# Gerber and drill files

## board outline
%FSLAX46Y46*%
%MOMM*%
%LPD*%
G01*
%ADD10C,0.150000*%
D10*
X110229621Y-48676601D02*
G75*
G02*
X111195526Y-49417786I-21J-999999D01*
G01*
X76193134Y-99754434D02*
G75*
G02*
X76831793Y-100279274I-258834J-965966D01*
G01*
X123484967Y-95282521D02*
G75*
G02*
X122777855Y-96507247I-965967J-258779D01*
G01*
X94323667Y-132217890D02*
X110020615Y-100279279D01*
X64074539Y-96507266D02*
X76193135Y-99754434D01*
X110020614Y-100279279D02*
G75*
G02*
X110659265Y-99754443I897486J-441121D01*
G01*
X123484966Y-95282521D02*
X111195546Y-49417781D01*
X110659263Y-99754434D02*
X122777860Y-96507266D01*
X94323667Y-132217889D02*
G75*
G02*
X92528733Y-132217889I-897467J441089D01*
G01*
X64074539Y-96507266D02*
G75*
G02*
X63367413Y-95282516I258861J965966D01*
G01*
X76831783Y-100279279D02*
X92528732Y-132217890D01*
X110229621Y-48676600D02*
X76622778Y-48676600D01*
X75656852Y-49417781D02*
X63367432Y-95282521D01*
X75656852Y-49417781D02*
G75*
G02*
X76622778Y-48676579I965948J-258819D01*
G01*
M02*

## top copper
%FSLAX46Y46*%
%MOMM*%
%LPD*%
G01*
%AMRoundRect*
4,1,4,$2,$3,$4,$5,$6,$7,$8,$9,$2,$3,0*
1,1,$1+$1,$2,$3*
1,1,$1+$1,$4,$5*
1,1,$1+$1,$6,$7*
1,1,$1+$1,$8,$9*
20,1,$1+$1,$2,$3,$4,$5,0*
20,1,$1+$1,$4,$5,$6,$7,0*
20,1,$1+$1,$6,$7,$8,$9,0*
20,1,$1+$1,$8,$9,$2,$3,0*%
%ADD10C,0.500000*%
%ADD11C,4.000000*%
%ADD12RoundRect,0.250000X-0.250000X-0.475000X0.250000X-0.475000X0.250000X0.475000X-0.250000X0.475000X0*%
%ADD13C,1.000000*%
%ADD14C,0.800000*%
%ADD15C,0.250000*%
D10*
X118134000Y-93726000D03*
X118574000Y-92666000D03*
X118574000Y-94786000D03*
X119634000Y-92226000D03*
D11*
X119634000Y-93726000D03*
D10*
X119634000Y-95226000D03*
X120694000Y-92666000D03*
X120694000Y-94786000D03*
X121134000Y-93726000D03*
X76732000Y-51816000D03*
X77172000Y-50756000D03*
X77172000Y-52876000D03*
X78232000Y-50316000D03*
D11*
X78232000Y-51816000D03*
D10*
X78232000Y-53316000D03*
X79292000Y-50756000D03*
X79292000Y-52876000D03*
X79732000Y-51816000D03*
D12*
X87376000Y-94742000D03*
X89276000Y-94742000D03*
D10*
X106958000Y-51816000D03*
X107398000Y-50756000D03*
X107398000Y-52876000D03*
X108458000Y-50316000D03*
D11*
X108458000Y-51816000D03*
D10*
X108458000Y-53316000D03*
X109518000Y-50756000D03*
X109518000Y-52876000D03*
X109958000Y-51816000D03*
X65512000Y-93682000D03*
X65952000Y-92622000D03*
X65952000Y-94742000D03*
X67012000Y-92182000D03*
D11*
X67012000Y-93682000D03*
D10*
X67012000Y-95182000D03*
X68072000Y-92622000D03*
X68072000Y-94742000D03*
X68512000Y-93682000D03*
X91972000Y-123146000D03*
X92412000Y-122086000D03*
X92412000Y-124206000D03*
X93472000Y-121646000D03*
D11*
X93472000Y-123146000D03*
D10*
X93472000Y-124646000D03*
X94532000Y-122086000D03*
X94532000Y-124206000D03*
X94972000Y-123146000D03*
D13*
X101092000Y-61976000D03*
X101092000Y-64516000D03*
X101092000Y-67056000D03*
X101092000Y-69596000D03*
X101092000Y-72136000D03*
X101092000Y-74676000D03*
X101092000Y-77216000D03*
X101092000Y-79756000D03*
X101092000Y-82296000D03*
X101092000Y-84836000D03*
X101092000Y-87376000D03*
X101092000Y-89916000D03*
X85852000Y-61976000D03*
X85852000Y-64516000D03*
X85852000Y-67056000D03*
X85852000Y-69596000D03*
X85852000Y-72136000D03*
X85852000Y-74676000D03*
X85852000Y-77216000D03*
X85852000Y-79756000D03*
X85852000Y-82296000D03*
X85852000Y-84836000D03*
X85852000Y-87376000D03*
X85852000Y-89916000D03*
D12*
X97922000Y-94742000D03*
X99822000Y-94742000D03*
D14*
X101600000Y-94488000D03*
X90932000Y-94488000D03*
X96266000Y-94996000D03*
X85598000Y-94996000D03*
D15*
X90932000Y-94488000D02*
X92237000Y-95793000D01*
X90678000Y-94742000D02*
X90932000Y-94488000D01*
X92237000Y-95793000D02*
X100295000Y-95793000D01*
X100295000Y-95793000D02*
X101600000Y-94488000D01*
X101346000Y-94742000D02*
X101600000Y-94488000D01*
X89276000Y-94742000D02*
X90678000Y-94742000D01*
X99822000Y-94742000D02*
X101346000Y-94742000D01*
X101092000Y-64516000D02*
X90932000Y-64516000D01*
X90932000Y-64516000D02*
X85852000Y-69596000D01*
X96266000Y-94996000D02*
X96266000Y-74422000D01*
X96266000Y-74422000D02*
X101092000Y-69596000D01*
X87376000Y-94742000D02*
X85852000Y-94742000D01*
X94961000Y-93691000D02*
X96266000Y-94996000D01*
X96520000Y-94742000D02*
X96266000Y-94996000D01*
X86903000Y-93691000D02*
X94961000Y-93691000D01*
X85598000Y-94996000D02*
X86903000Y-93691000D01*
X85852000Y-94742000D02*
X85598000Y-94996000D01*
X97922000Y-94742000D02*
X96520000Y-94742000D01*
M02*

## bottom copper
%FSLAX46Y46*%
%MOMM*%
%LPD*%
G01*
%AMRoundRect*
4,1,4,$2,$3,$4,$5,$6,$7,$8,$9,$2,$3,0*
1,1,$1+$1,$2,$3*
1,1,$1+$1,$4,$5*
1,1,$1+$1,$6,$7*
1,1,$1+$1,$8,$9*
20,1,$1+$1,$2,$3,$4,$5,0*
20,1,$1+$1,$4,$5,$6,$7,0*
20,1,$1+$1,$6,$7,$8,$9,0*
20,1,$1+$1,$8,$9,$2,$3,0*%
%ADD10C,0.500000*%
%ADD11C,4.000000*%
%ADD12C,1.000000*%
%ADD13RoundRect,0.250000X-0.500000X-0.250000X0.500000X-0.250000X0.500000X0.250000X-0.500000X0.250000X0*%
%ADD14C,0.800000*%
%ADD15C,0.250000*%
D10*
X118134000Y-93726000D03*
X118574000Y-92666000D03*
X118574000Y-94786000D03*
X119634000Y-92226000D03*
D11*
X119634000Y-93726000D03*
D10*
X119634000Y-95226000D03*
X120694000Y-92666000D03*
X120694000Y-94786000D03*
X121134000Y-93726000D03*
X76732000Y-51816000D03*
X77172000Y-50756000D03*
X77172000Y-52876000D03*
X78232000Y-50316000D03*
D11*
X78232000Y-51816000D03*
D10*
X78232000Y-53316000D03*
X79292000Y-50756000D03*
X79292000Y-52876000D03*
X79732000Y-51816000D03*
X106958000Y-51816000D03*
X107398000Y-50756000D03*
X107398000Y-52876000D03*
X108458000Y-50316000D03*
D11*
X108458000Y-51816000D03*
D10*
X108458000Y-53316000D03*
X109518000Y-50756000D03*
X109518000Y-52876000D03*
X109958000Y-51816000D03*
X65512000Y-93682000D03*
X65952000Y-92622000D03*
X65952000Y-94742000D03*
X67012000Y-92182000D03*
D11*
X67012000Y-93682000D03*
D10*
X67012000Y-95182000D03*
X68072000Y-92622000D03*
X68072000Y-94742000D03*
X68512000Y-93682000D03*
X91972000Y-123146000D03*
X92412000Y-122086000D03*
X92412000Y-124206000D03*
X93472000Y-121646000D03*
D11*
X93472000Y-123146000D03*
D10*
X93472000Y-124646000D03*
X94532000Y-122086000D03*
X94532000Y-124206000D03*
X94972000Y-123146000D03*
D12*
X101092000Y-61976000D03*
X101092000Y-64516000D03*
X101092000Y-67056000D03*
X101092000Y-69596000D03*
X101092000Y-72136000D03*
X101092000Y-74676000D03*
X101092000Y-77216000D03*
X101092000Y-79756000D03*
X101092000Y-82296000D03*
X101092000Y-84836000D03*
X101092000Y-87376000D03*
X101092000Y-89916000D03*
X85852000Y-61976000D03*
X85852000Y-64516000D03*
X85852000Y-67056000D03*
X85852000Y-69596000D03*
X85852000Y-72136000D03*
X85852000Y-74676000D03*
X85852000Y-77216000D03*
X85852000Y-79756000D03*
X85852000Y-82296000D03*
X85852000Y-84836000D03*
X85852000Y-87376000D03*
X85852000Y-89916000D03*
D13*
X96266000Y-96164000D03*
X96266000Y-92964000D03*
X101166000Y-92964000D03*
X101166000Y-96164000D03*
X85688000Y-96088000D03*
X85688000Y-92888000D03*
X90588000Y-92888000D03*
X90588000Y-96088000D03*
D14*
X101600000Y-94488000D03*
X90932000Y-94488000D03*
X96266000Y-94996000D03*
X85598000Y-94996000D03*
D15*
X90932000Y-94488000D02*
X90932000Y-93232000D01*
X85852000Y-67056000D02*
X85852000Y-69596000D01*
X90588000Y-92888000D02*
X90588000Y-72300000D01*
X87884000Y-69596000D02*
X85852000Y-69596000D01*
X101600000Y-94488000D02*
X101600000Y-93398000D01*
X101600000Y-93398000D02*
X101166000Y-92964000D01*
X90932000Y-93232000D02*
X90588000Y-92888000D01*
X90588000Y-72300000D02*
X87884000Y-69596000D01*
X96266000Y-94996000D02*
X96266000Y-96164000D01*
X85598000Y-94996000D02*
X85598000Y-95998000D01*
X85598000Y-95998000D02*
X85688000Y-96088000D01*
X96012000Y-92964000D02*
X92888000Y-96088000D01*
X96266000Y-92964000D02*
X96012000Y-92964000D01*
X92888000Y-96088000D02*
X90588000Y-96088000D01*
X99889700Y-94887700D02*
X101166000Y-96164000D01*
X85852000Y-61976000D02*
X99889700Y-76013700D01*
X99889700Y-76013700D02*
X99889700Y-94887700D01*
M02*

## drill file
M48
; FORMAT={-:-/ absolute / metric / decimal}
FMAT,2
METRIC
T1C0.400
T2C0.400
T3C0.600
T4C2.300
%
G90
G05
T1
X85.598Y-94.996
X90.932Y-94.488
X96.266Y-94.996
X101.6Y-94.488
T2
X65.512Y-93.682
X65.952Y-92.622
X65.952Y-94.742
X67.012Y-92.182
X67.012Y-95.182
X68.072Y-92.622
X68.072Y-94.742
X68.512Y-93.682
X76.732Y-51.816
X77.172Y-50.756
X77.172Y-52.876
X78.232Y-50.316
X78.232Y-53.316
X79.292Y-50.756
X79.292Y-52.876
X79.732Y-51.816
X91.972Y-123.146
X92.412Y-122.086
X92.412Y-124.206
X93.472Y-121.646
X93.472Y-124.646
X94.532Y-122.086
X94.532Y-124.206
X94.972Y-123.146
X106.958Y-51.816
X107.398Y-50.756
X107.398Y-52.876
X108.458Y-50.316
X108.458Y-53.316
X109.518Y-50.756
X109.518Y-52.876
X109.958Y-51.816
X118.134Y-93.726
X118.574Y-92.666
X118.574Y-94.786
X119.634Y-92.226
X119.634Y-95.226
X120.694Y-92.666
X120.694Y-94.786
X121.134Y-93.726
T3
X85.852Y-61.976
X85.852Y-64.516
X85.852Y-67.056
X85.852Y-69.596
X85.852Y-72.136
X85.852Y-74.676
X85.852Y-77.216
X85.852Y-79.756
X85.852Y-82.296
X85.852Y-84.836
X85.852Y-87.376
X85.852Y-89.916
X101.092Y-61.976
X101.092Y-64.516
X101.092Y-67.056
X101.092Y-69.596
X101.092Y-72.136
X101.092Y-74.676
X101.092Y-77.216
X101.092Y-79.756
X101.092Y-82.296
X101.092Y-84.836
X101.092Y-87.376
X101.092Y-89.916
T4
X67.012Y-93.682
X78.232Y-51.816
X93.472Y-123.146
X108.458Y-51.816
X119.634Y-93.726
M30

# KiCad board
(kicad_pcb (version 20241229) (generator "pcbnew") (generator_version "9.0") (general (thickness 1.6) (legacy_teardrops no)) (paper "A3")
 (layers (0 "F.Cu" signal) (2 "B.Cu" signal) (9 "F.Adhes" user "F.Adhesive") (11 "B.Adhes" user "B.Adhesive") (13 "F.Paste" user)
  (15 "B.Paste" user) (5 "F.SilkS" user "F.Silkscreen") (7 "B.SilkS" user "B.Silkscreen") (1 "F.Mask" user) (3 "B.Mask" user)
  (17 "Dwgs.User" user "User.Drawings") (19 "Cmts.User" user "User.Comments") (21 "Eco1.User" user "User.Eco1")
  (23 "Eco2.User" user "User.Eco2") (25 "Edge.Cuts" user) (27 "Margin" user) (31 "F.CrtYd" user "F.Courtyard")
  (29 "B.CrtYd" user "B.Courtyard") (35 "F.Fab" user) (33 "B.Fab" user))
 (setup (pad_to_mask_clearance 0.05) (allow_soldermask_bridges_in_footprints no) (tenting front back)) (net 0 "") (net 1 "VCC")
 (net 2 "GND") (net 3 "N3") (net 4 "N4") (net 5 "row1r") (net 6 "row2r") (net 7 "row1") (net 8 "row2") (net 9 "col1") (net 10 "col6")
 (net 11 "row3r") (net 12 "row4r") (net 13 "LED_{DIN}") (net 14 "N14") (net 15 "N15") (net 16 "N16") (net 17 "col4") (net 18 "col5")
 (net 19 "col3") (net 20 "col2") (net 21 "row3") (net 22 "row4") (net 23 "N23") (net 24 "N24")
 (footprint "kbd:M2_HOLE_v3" (layer "F.Cu") (at 119.634 93.726)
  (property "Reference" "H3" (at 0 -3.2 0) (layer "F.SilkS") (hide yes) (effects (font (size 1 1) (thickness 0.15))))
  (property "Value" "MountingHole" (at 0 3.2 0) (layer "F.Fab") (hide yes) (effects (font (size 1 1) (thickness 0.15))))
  (pad "1" thru_hole circle (at -1.5 0) (size 0.5 0.5) (drill 0.4) (layers "*.Cu" "*.Mask") (remove_unused_layers no))
  (pad "1" thru_hole circle (at -1.06 -1.06) (size 0.5 0.5) (drill 0.4) (layers "*.Cu" "*.Mask") (remove_unused_layers no))
  (pad "1" thru_hole circle (at -1.06 1.06) (size 0.5 0.5) (drill 0.4) (layers "*.Cu" "*.Mask") (remove_unused_layers no))
  (pad "1" thru_hole circle (at 0 -1.5) (size 0.5 0.5) (drill 0.4) (layers "*.Cu" "*.Mask") (remove_unused_layers no))
  (pad "1" thru_hole circle (at 0 0) (size 4 4) (drill 2.3) (layers "*.Cu" "*.Mask") (remove_unused_layers no))
  (pad "1" thru_hole circle (at 0 1.5) (size 0.5 0.5) (drill 0.4) (layers "*.Cu" "*.Mask") (remove_unused_layers no))
  (pad "1" thru_hole circle (at 1.06 -1.06) (size 0.5 0.5) (drill 0.4) (layers "*.Cu" "*.Mask") (remove_unused_layers no))
  (pad "1" thru_hole circle (at 1.06 1.06) (size 0.5 0.5) (drill 0.4) (layers "*.Cu" "*.Mask") (remove_unused_layers no))
  (pad "1" thru_hole circle (at 1.5 0) (size 0.5 0.5) (drill 0.4) (layers "*.Cu" "*.Mask") (remove_unused_layers no)))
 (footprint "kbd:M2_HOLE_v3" (layer "F.Cu") (at 78.232 51.816)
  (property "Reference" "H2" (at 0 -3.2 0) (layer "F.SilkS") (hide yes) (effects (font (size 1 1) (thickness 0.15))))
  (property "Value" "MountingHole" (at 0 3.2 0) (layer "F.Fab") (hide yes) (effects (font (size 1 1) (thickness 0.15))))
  (pad "1" thru_hole circle (at -1.5 0) (size 0.5 0.5) (drill 0.4) (layers "*.Cu" "*.Mask") (remove_unused_layers no))
  (pad "1" thru_hole circle (at -1.06 -1.06) (size 0.5 0.5) (drill 0.4) (layers "*.Cu" "*.Mask") (remove_unused_layers no))
  (pad "1" thru_hole circle (at -1.06 1.06) (size 0.5 0.5) (drill 0.4) (layers "*.Cu" "*.Mask") (remove_unused_layers no))
  (pad "1" thru_hole circle (at 0 -1.5) (size 0.5 0.5) (drill 0.4) (layers "*.Cu" "*.Mask") (remove_unused_layers no))
  (pad "1" thru_hole circle (at 0 0) (size 4 4) (drill 2.3) (layers "*.Cu" "*.Mask") (remove_unused_layers no))
  (pad "1" thru_hole circle (at 0 1.5) (size 0.5 0.5) (drill 0.4) (layers "*.Cu" "*.Mask") (remove_unused_layers no))
  (pad "1" thru_hole circle (at 1.06 -1.06) (size 0.5 0.5) (drill 0.4) (layers "*.Cu" "*.Mask") (remove_unused_layers no))
  (pad "1" thru_hole circle (at 1.06 1.06) (size 0.5 0.5) (drill 0.4) (layers "*.Cu" "*.Mask") (remove_unused_layers no))
  (pad "1" thru_hole circle (at 1.5 0) (size 0.5 0.5) (drill 0.4) (layers "*.Cu" "*.Mask") (remove_unused_layers no)))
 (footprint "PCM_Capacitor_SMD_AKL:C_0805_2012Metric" (layer "F.Cu") (at 88.326 94.742)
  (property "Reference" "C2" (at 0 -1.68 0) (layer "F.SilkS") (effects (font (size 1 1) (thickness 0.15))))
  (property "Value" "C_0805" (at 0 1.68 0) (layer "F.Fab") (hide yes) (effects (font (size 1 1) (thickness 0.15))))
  (pad "1" smd roundrect (at -0.95 0) (size 1 1.45) (layers "F.Cu" "F.Mask" "F.Paste") (roundrect_rratio 0.25) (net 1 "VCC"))
  (pad "2" smd roundrect (at 0.95 0) (size 1 1.45) (layers "F.Cu" "F.Mask" "F.Paste") (roundrect_rratio 0.25) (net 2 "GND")))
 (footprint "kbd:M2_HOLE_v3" (layer "F.Cu") (at 108.458 51.816)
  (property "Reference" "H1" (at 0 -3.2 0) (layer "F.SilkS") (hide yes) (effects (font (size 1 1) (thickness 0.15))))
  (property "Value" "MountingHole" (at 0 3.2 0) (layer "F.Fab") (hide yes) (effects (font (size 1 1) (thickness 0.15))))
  (pad "1" thru_hole circle (at -1.5 0) (size 0.5 0.5) (drill 0.4) (layers "*.Cu" "*.Mask") (remove_unused_layers no))
  (pad "1" thru_hole circle (at -1.06 -1.06) (size 0.5 0.5) (drill 0.4) (layers "*.Cu" "*.Mask") (remove_unused_layers no))
  (pad "1" thru_hole circle (at -1.06 1.06) (size 0.5 0.5) (drill 0.4) (layers "*.Cu" "*.Mask") (remove_unused_layers no))
  (pad "1" thru_hole circle (at 0 -1.5) (size 0.5 0.5) (drill 0.4) (layers "*.Cu" "*.Mask") (remove_unused_layers no))
  (pad "1" thru_hole circle (at 0 0) (size 4 4) (drill 2.3) (layers "*.Cu" "*.Mask") (remove_unused_layers no))
  (pad "1" thru_hole circle (at 0 1.5) (size 0.5 0.5) (drill 0.4) (layers "*.Cu" "*.Mask") (remove_unused_layers no))
  (pad "1" thru_hole circle (at 1.06 -1.06) (size 0.5 0.5) (drill 0.4) (layers "*.Cu" "*.Mask") (remove_unused_layers no))
  (pad "1" thru_hole circle (at 1.06 1.06) (size 0.5 0.5) (drill 0.4) (layers "*.Cu" "*.Mask") (remove_unused_layers no))
  (pad "1" thru_hole circle (at 1.5 0) (size 0.5 0.5) (drill 0.4) (layers "*.Cu" "*.Mask") (remove_unused_layers no)))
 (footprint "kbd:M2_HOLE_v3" (layer "F.Cu") (at 67.012 93.682)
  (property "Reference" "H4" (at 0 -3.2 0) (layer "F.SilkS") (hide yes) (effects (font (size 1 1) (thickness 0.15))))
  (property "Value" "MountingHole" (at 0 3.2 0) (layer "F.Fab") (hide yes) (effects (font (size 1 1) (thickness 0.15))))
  (pad "1" thru_hole circle (at -1.5 0) (size 0.5 0.5) (drill 0.4) (layers "*.Cu" "*.Mask") (remove_unused_layers no))
  (pad "1" thru_hole circle (at -1.06 -1.06) (size 0.5 0.5) (drill 0.4) (layers "*.Cu" "*.Mask") (remove_unused_layers no))
  (pad "1" thru_hole circle (at -1.06 1.06) (size 0.5 0.5) (drill 0.4) (layers "*.Cu" "*.Mask") (remove_unused_layers no))
  (pad "1" thru_hole circle (at 0 -1.5) (size 0.5 0.5) (drill 0.4) (layers "*.Cu" "*.Mask") (remove_unused_layers no))
  (pad "1" thru_hole circle (at 0 0) (size 4 4) (drill 2.3) (layers "*.Cu" "*.Mask") (remove_unused_layers no))
  (pad "1" thru_hole circle (at 0 1.5) (size 0.5 0.5) (drill 0.4) (layers "*.Cu" "*.Mask") (remove_unused_layers no))
  (pad "1" thru_hole circle (at 1.06 -1.06) (size 0.5 0.5) (drill 0.4) (layers "*.Cu" "*.Mask") (remove_unused_layers no))
  (pad "1" thru_hole circle (at 1.06 1.06) (size 0.5 0.5) (drill 0.4) (layers "*.Cu" "*.Mask") (remove_unused_layers no))
  (pad "1" thru_hole circle (at 1.5 0) (size 0.5 0.5) (drill 0.4) (layers "*.Cu" "*.Mask") (remove_unused_layers no)))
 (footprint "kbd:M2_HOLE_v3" (layer "F.Cu") (at 93.472 123.146)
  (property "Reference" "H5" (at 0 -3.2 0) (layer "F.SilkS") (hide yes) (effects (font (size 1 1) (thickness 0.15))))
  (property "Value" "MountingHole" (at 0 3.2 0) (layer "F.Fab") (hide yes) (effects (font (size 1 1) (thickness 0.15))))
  (pad "1" thru_hole circle (at -1.5 0) (size 0.5 0.5) (drill 0.4) (layers "*.Cu" "*.Mask") (remove_unused_layers no))
  (pad "1" thru_hole circle (at -1.06 -1.06) (size 0.5 0.5) (drill 0.4) (layers "*.Cu" "*.Mask") (remove_unused_layers no))
  (pad "1" thru_hole circle (at -1.06 1.06) (size 0.5 0.5) (drill 0.4) (layers "*.Cu" "*.Mask") (remove_unused_layers no))
  (pad "1" thru_hole circle (at 0 -1.5) (size 0.5 0.5) (drill 0.4) (layers "*.Cu" "*.Mask") (remove_unused_layers no))
  (pad "1" thru_hole circle (at 0 0) (size 4 4) (drill 2.3) (layers "*.Cu" "*.Mask") (remove_unused_layers no))
  (pad "1" thru_hole circle (at 0 1.5) (size 0.5 0.5) (drill 0.4) (layers "*.Cu" "*.Mask") (remove_unused_layers no))
  (pad "1" thru_hole circle (at 1.06 -1.06) (size 0.5 0.5) (drill 0.4) (layers "*.Cu" "*.Mask") (remove_unused_layers no))
  (pad "1" thru_hole circle (at 1.06 1.06) (size 0.5 0.5) (drill 0.4) (layers "*.Cu" "*.Mask") (remove_unused_layers no))
  (pad "1" thru_hole circle (at 1.5 0) (size 0.5 0.5) (drill 0.4) (layers "*.Cu" "*.Mask") (remove_unused_layers no)))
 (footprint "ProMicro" (layer "F.Cu") (at 93.472 75.946 -90)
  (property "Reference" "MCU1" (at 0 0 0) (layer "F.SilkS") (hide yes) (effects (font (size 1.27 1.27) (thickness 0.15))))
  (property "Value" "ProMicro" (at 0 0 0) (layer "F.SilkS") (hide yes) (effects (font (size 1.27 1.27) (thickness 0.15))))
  (pad "1" thru_hole circle (at -13.97 -7.62) (size 1 1) (drill 0.6) (layers "*.Cu" "F.Mask" "F.SilkS") (remove_unused_layers no)
   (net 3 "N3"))
  (pad "2" thru_hole circle (at -11.43 -7.62) (size 1 1) (drill 0.6) (layers "*.Cu" "F.Mask" "F.SilkS") (remove_unused_layers no)
   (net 2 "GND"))
  (pad "3" thru_hole circle (at -8.89 -7.62) (size 1 1) (drill 0.6) (layers "*.Cu" "F.Mask" "F.SilkS") (remove_unused_layers no)
   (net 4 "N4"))
  (pad "4" thru_hole circle (at -6.35 -7.62) (size 1 1) (drill 0.6) (layers "*.Cu" "F.Mask" "F.SilkS") (remove_unused_layers no)
   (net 1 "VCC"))
  (pad "5" thru_hole circle (at -3.81 -7.62) (size 1 1) (drill 0.6) (layers "*.Cu" "F.Mask" "F.SilkS") (remove_unused_layers no)
   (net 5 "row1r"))
  (pad "6" thru_hole circle (at -1.27 -7.62) (size 1 1) (drill 0.6) (layers "*.Cu" "F.Mask" "F.SilkS") (remove_unused_layers no)
   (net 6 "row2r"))
  (pad "7" thru_hole circle (at 1.27 -7.62) (size 1 1) (drill 0.6) (layers "*.Cu" "F.Mask" "F.SilkS") (remove_unused_layers no)
   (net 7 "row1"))
  (pad "8" thru_hole circle (at 3.81 -7.62) (size 1 1) (drill 0.6) (layers "*.Cu" "F.Mask" "F.SilkS") (remove_unused_layers no)
   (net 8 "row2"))
  (pad "9" thru_hole circle (at 6.35 -7.62) (size 1 1) (drill 0.6) (layers "*.Cu" "F.Mask" "F.SilkS") (remove_unused_layers no)
   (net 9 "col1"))
  (pad "10" thru_hole circle (at 8.89 -7.62) (size 1 1) (drill 0.6) (layers "*.Cu" "F.Mask" "F.SilkS") (remove_unused_layers no)
   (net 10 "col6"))
  (pad "11" thru_hole circle (at 11.43 -7.62) (size 1 1) (drill 0.6) (layers "*.Cu" "F.Mask" "F.SilkS") (remove_unused_layers no)
   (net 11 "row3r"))
  (pad "12" thru_hole circle (at 13.97 -7.62) (size 1 1) (drill 0.6) (layers "*.Cu" "F.Mask" "F.SilkS") (remove_unused_layers no)
   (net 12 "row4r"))
  (pad "13" thru_hole circle (at -13.97 7.62) (size 1 1) (drill 0.6) (layers "*.Cu" "F.Mask" "F.SilkS") (remove_unused_layers no)
   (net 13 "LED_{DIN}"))
  (pad "14" thru_hole circle (at -11.43 7.62) (size 1 1) (drill 0.6) (layers "*.Cu" "F.Mask" "F.SilkS") (remove_unused_layers no)
   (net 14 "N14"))
  (pad "15" thru_hole circle (at -8.89 7.62) (size 1 1) (drill 0.6) (layers "*.Cu" "F.Mask" "F.SilkS") (remove_unused_layers no)
   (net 2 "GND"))
  (pad "16" thru_hole circle (at -6.35 7.62) (size 1 1) (drill 0.6) (layers "*.Cu" "F.Mask" "F.SilkS") (remove_unused_layers no)
   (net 2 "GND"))
  (pad "17" thru_hole circle (at -3.81 7.62) (size 1 1) (drill 0.6) (layers "*.Cu" "F.Mask" "F.SilkS") (remove_unused_layers no)
   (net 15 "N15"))
  (pad "18" thru_hole circle (at -1.27 7.62) (size 1 1) (drill 0.6) (layers "*.Cu" "F.Mask" "F.SilkS") (remove_unused_layers no)
   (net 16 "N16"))
  (pad "19" thru_hole circle (at 1.27 7.62) (size 1 1) (drill 0.6) (layers "*.Cu" "F.Mask" "F.SilkS") (remove_unused_layers no)
   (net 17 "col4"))
  (pad "20" thru_hole circle (at 3.81 7.62) (size 1 1) (drill 0.6) (layers "*.Cu" "F.Mask" "F.SilkS") (remove_unused_layers no)
   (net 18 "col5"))
  (pad "21" thru_hole circle (at 6.35 7.62) (size 1 1) (drill 0.6) (layers "*.Cu" "F.Mask" "F.SilkS") (remove_unused_layers no)
   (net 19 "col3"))
  (pad "22" thru_hole circle (at 8.89 7.62) (size 1 1) (drill 0.6) (layers "*.Cu" "F.Mask" "F.SilkS") (remove_unused_layers no)
   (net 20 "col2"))
  (pad "23" thru_hole circle (at 11.43 7.62) (size 1 1) (drill 0.6) (layers "*.Cu" "F.Mask" "F.SilkS") (remove_unused_layers no)
   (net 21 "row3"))
  (pad "24" thru_hole circle (at 13.97 7.62) (size 1 1) (drill 0.6) (layers "*.Cu" "F.Mask" "F.SilkS") (remove_unused_layers no)
   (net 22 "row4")))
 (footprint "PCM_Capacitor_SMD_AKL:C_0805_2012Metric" (layer "F.Cu") (at 98.872 94.742)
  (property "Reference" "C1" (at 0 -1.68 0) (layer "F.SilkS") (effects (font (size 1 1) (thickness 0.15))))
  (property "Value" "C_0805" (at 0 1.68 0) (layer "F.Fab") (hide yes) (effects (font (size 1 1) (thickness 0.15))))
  (pad "1" smd roundrect (at -0.95 0) (size 1 1.45) (layers "F.Cu" "F.Mask" "F.Paste") (roundrect_rratio 0.25) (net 1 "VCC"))
  (pad "2" smd roundrect (at 0.95 0) (size 1 1.45) (layers "F.Cu" "F.Mask" "F.Paste") (roundrect_rratio 0.25) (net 2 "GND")))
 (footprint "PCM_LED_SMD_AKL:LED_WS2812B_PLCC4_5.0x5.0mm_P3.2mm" (layer "B.Cu") (at 98.716 94.564)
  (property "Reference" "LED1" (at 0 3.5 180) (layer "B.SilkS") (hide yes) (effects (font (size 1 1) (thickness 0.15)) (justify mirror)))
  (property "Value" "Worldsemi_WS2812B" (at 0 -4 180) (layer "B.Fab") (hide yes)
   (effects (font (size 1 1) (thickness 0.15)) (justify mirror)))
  (pad "1" smd roundrect (at -2.45 1.6) (size 1.5 1) (layers "B.Cu" "B.Mask" "B.Paste") (roundrect_rratio 0.25) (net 1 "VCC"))
  (pad "2" smd roundrect (at -2.45 -1.6) (size 1.5 1) (layers "B.Cu" "B.Mask" "B.Paste") (roundrect_rratio 0.25) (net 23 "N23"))
  (pad "3" smd roundrect (at 2.45 -1.6) (size 1.5 1) (layers "B.Cu" "B.Mask" "B.Paste") (roundrect_rratio 0.25) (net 2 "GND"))
  (pad "4" smd roundrect (at 2.45 1.6) (size 1.5 1) (layers "B.Cu" "B.Mask" "B.Paste") (roundrect_rratio 0.25) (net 13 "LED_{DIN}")))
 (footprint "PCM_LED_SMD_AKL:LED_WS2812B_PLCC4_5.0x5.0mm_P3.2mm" (layer "B.Cu") (at 88.138 94.488)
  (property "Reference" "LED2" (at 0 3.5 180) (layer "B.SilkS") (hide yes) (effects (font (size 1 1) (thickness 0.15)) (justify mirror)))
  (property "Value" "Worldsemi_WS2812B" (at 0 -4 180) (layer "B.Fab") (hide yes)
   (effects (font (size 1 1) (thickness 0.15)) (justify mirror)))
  (pad "1" smd roundrect (at -2.45 1.6) (size 1.5 1) (layers "B.Cu" "B.Mask" "B.Paste") (roundrect_rratio 0.25) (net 1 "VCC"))
  (pad "2" smd roundrect (at -2.45 -1.6) (size 1.5 1) (layers "B.Cu" "B.Mask" "B.Paste") (roundrect_rratio 0.25) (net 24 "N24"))
  (pad "3" smd roundrect (at 2.45 -1.6) (size 1.5 1) (layers "B.Cu" "B.Mask" "B.Paste") (roundrect_rratio 0.25) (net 2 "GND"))
  (pad "4" smd roundrect (at 2.45 1.6) (size 1.5 1) (layers "B.Cu" "B.Mask" "B.Paste") (roundrect_rratio 0.25) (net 23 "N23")))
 (gr_arc (start 110.229621 48.676601) (mid 110.838382 48.883247) (end 111.195546 49.417781) (stroke (width 0.15) (type solid))
  (layer "Edge.Cuts"))
 (gr_arc (start 76.193134 99.754434) (mid 76.569229 99.947776) (end 76.831783 100.279279) (stroke (width 0.15) (type solid))
  (layer "Edge.Cuts"))
 (gr_arc (start 123.484967 95.282521) (mid 123.385066 96.04134) (end 122.77786 96.507266) (stroke (width 0.15) (type solid))
  (layer "Edge.Cuts"))
 (gr_line (start 94.323667 132.21789) (end 110.020615 100.279279) (stroke (width 0.15) (type solid)) (layer "Edge.Cuts"))
 (gr_line (start 64.074539 96.507266) (end 76.193135 99.754434) (stroke (width 0.15) (type solid)) (layer "Edge.Cuts"))
 (gr_arc (start 110.020614 100.279279) (mid 110.283168 99.947776) (end 110.659263 99.754434) (stroke (width 0.15) (type solid))
  (layer "Edge.Cuts"))
 (gr_line (start 123.484966 95.282521) (end 111.195546 49.417781) (stroke (width 0.15) (type solid)) (layer "Edge.Cuts"))
 (gr_line (start 110.659263 99.754434) (end 122.77786 96.507266) (stroke (width 0.15) (type solid)) (layer "Edge.Cuts"))
 (gr_arc (start 94.323667 132.217889) (mid 93.4262 132.776809) (end 92.528732 132.21789) (stroke (width 0.15) (type solid))
  (layer "Edge.Cuts"))
 (gr_arc (start 64.074539 96.507266) (mid 63.467333 96.04134) (end 63.367432 95.282521) (stroke (width 0.15) (type solid))
  (layer "Edge.Cuts"))
 (gr_line (start 76.831783 100.279279) (end 92.528732 132.21789) (stroke (width 0.15) (type solid)) (layer "Edge.Cuts"))
 (gr_line (start 110.229621 48.6766) (end 76.622778 48.6766) (stroke (width 0.15) (type solid)) (layer "Edge.Cuts"))
 (gr_line (start 75.656852 49.417781) (end 63.367432 95.282521) (stroke (width 0.15) (type solid)) (layer "Edge.Cuts"))
 (gr_arc (start 75.656852 49.417781) (mid 76.014016 48.883247) (end 76.622778 48.6766) (stroke (width 0.15) (type solid))
  (layer "Edge.Cuts"))
 (segment (start 90.932 94.488) (end 92.237 95.793) (width 0.25) (layer "F.Cu") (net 2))
 (segment (start 90.678 94.742) (end 90.932 94.488) (width 0.25) (layer "F.Cu") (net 2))
 (segment (start 92.237 95.793) (end 100.295 95.793) (width 0.25) (layer "F.Cu") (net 2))
 (segment (start 100.295 95.793) (end 101.6 94.488) (width 0.25) (layer "F.Cu") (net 2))
 (segment (start 101.346 94.742) (end 101.6 94.488) (width 0.25) (layer "F.Cu") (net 2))
 (segment (start 89.276 94.742) (end 90.678 94.742) (width 0.25) (layer "F.Cu") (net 2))
 (segment (start 99.822 94.742) (end 101.346 94.742) (width 0.25) (layer "F.Cu") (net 2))
 (segment (start 101.092 64.516) (end 90.932 64.516) (width 0.25) (layer "F.Cu") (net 2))
 (segment (start 90.932 64.516) (end 85.852 69.596) (width 0.25) (layer "F.Cu") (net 2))
 (via (at 101.6 94.488) (size 0.8) (drill 0.4) (layers "F.Cu" "B.Cu") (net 2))
 (via (at 90.932 94.488) (size 0.8) (drill 0.4) (layers "F.Cu" "B.Cu") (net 2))
 (segment (start 90.932 94.488) (end 90.932 93.232) (width 0.25) (layer "B.Cu") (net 2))
 (segment (start 85.852 67.056) (end 85.852 69.596) (width 0.25) (layer "B.Cu") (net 2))
 (segment (start 90.588 92.888) (end 90.588 72.3) (width 0.25) (layer "B.Cu") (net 2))
 (segment (start 87.884 69.596) (end 85.852 69.596) (width 0.25) (layer "B.Cu") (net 2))
 (segment (start 101.6 94.488) (end 101.6 93.398) (width 0.25) (layer "B.Cu") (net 2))
 (segment (start 101.6 93.398) (end 101.166 92.964) (width 0.25) (layer "B.Cu") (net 2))
 (segment (start 90.932 93.232) (end 90.588 92.888) (width 0.25) (layer "B.Cu") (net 2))
 (segment (start 90.588 72.3) (end 87.884 69.596) (width 0.25) (layer "B.Cu") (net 2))
 (segment (start 96.266 94.996) (end 96.266 74.422) (width 0.25) (layer "F.Cu") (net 1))
 (segment (start 96.266 74.422) (end 101.092 69.596) (width 0.25) (layer "F.Cu") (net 1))
 (segment (start 87.376 94.742) (end 85.852 94.742) (width 0.25) (layer "F.Cu") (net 1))
 (segment (start 94.961 93.691) (end 96.266 94.996) (width 0.25) (layer "F.Cu") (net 1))
 (segment (start 96.52 94.742) (end 96.266 94.996) (width 0.25) (layer "F.Cu") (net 1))
 (segment (start 86.903 93.691) (end 94.961 93.691) (width 0.25) (layer "F.Cu") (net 1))
 (segment (start 85.598 94.996) (end 86.903 93.691) (width 0.25) (layer "F.Cu") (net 1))
 (segment (start 85.852 94.742) (end 85.598 94.996) (width 0.25) (layer "F.Cu") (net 1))
 (segment (start 97.922 94.742) (end 96.52 94.742) (width 0.25) (layer "F.Cu") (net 1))
 (via (at 96.266 94.996) (size 0.8) (drill 0.4) (layers "F.Cu" "B.Cu") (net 1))
 (via (at 85.598 94.996) (size 0.8) (drill 0.4) (layers "F.Cu" "B.Cu") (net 1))
 (segment (start 96.266 94.996) (end 96.266 96.164) (width 0.25) (layer "B.Cu") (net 1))
 (segment (start 85.598 94.996) (end 85.598 95.998) (width 0.25) (layer "B.Cu") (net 1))
 (segment (start 85.598 95.998) (end 85.688 96.088) (width 0.25) (layer "B.Cu") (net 1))
 (segment (start 96.012 92.964) (end 92.888 96.088) (width 0.25) (layer "B.Cu") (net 23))
 (segment (start 96.266 92.964) (end 96.012 92.964) (width 0.25) (layer "B.Cu") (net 23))
 (segment (start 92.888 96.088) (end 90.588 96.088) (width 0.25) (layer "B.Cu") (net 23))
 (segment (start 99.8897 94.8877) (end 101.166 96.164) (width 0.25) (layer "B.Cu") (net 13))
 (segment (start 85.852 61.976) (end 99.8897 76.0137) (width 0.25) (layer "B.Cu") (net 13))
 (segment (start 99.8897 76.0137) (end 99.8897 94.8877) (width 0.25) (layer "B.Cu") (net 13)))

